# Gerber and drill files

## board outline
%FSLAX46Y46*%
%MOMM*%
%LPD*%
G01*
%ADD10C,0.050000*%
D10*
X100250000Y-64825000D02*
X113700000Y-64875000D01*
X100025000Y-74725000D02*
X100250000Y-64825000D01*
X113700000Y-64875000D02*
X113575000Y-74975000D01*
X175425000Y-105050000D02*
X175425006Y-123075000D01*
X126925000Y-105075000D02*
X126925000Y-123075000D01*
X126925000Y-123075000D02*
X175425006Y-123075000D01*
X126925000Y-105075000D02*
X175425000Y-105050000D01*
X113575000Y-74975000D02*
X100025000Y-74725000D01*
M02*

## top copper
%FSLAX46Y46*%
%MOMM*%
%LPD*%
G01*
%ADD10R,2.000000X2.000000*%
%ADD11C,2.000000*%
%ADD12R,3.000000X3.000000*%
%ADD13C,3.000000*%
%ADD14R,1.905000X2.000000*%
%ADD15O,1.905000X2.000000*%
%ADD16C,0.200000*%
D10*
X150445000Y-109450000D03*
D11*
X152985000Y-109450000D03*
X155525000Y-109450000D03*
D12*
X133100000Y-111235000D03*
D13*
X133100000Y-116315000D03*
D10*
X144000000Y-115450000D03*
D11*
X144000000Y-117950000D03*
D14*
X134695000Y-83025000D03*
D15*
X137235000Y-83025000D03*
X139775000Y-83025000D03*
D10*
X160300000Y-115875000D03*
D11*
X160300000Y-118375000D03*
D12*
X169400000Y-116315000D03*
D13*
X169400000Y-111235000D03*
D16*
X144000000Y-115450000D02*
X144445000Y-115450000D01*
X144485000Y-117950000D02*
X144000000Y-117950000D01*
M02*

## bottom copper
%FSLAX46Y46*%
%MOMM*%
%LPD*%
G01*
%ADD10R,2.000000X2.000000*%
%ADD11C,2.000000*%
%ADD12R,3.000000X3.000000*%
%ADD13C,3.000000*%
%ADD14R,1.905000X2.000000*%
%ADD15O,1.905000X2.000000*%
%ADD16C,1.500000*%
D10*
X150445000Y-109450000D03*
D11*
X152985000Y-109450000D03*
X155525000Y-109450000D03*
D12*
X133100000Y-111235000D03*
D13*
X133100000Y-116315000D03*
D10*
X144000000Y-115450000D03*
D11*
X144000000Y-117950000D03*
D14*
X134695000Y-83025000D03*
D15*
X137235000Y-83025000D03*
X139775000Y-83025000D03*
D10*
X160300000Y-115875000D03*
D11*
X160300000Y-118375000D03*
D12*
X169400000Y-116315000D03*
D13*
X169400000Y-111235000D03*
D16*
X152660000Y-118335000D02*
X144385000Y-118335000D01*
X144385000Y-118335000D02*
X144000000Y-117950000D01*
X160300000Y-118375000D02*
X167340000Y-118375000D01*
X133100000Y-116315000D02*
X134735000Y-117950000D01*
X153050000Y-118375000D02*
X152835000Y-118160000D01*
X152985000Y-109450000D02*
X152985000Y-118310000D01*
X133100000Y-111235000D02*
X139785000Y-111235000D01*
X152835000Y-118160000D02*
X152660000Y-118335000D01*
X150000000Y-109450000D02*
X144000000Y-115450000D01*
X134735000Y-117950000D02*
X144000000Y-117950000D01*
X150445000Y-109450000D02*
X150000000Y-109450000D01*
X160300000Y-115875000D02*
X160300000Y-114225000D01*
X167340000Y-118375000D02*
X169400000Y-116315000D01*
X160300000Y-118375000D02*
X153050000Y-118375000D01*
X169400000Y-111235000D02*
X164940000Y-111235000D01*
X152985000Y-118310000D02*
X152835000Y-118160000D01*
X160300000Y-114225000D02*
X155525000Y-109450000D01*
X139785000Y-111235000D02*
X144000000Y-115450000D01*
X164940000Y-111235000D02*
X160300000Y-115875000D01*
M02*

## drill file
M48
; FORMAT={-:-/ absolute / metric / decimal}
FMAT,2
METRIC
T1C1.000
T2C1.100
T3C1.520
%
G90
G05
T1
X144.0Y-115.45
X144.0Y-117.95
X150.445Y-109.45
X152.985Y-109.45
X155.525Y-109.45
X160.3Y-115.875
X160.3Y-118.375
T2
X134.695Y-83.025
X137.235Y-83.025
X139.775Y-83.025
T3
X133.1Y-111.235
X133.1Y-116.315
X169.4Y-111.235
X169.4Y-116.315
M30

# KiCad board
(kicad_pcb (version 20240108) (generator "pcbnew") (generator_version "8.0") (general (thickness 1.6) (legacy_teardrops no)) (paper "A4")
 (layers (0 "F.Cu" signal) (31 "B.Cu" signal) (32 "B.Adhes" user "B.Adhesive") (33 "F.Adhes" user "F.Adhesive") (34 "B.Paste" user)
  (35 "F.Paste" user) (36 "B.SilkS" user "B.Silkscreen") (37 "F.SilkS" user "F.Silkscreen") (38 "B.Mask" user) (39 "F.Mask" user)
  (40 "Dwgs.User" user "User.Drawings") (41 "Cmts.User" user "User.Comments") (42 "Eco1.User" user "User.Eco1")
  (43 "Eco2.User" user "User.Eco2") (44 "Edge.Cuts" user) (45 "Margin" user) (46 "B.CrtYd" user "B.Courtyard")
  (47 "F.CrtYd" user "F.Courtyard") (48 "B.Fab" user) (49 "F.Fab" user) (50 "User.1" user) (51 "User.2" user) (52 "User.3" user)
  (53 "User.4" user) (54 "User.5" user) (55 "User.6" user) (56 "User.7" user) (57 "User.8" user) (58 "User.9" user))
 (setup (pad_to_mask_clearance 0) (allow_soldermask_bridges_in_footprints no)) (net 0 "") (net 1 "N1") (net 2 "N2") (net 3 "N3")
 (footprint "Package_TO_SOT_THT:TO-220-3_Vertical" (layer "F.Cu") (at 150.445 109.45)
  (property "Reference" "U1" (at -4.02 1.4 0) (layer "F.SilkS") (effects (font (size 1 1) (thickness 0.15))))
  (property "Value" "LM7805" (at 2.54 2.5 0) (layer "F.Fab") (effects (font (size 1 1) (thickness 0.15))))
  (pad "1" thru_hole rect (at 0 0) (size 2 2) (drill 1) (layers "*.Cu" "*.Mask") (remove_unused_layers no))
  (pad "2" thru_hole circle (at 2.54 0) (size 2 2) (drill 1) (layers "*.Cu" "*.Mask") (remove_unused_layers no))
  (pad "3" thru_hole circle (at 5.08 0) (size 2 2) (drill 1) (layers "*.Cu" "*.Mask") (remove_unused_layers no)))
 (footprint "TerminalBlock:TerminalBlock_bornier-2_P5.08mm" (layer "F.Cu") (at 133.1 111.235 -90)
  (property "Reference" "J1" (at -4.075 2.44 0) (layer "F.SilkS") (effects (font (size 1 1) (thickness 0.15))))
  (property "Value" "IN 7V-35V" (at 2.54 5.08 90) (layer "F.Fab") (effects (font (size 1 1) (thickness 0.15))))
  (pad "1" thru_hole rect (at 0 0 270) (size 3 3) (drill 1.52) (layers "*.Cu" "*.Mask") (remove_unused_layers no))
  (pad "2" thru_hole circle (at 5.08 0 270) (size 3 3) (drill 1.52) (layers "*.Cu" "*.Mask") (remove_unused_layers no)))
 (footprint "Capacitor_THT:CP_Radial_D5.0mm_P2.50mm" (layer "F.Cu") (at 144 115.45 -90)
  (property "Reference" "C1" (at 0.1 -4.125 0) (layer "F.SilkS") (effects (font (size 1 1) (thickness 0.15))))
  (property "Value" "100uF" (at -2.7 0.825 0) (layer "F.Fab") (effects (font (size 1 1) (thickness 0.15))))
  (pad "1" thru_hole rect (at 0 0 270) (size 2 2) (drill 1) (layers "*.Cu" "*.Mask") (remove_unused_layers no))
  (pad "2" thru_hole circle (at 2.5 0 270) (size 2 2) (drill 1) (layers "*.Cu" "*.Mask") (remove_unused_layers no)))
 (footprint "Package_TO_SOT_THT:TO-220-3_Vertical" (layer "F.Cu") (at 134.695 83.025)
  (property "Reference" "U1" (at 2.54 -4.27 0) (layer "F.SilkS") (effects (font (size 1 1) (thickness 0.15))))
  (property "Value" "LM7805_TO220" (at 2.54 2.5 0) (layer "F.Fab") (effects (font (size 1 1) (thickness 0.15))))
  (pad "1" thru_hole rect (at 0 0) (size 1.905 2) (drill 1.1) (layers "*.Cu" "*.Mask") (remove_unused_layers no) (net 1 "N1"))
  (pad "2" thru_hole oval (at 2.54 0) (size 1.905 2) (drill 1.1) (layers "*.Cu" "*.Mask") (remove_unused_layers no) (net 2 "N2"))
  (pad "3" thru_hole oval (at 5.08 0) (size 1.905 2) (drill 1.1) (layers "*.Cu" "*.Mask") (remove_unused_layers no) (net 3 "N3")))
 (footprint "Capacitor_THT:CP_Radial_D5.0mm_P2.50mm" (layer "F.Cu") (at 160.3 115.875 -90)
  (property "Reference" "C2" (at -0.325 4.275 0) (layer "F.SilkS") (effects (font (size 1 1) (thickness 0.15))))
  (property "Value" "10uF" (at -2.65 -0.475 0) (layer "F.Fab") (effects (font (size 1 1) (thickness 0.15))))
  (pad "1" thru_hole rect (at 0 0 270) (size 2 2) (drill 1) (layers "*.Cu" "*.Mask") (remove_unused_layers no))
  (pad "2" thru_hole circle (at 2.5 0 270) (size 2 2) (drill 1) (layers "*.Cu" "*.Mask") (remove_unused_layers no)))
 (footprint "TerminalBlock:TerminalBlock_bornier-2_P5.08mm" (layer "F.Cu") (at 169.4 116.315 90)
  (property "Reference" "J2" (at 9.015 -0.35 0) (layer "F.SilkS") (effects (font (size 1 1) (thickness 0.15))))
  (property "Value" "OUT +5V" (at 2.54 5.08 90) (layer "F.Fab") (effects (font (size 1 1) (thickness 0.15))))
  (pad "1" thru_hole rect (at 0 0 90) (size 3 3) (drill 1.52) (layers "*.Cu" "*.Mask") (remove_unused_layers no))
  (pad "2" thru_hole circle (at 5.08 0 90) (size 3 3) (drill 1.52) (layers "*.Cu" "*.Mask") (remove_unused_layers no)))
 (gr_line (start 100.25 64.825) (end 113.7 64.875) (stroke (width 0.05) (type default)) (layer "Edge.Cuts"))
 (gr_line (start 100.025 74.725) (end 100.25 64.825) (stroke (width 0.05) (type default)) (layer "Edge.Cuts"))
 (gr_line (start 113.7 64.875) (end 113.575 74.975) (stroke (width 0.05) (type default)) (layer "Edge.Cuts"))
 (gr_line (start 175.425 105.05) (end 175.425006 123.075) (stroke (width 0.05) (type default)) (layer "Edge.Cuts"))
 (gr_line (start 126.925 105.075) (end 126.925 123.075) (stroke (width 0.05) (type default)) (layer "Edge.Cuts"))
 (gr_line (start 126.925 123.075) (end 175.425006 123.075) (stroke (width 0.05) (type default)) (layer "Edge.Cuts"))
 (gr_line (start 126.925 105.075) (end 175.425 105.05) (stroke (width 0.05) (type default)) (layer "Edge.Cuts"))
 (gr_line (start 113.575 74.975) (end 100.025 74.725) (stroke (width 0.05) (type default)) (layer "Edge.Cuts"))
 (segment (start 144 115.45) (end 144.445 115.45) (width 0.2) (layer "F.Cu") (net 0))
 (segment (start 144.485 117.95) (end 144 117.95) (width 0.2) (layer "F.Cu") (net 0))
 (segment (start 152.66 118.335) (end 144.385 118.335) (width 1.5) (layer "B.Cu") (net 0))
 (segment (start 144.385 118.335) (end 144 117.95) (width 1.5) (layer "B.Cu") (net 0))
 (segment (start 160.3 118.375) (end 167.34 118.375) (width 1.5) (layer "B.Cu") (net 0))
 (segment (start 133.1 116.315) (end 134.735 117.95) (width 1.5) (layer "B.Cu") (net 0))
 (segment (start 153.05 118.375) (end 152.835 118.16) (width 1.5) (layer "B.Cu") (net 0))
 (segment (start 152.985 109.45) (end 152.985 118.31) (width 1.5) (layer "B.Cu") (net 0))
 (segment (start 133.1 111.235) (end 139.785 111.235) (width 1.5) (layer "B.Cu") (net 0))
 (segment (start 152.835 118.16) (end 152.66 118.335) (width 1.5) (layer "B.Cu") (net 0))
 (segment (start 150 109.45) (end 144 115.45) (width 1.5) (layer "B.Cu") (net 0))
 (segment (start 134.735 117.95) (end 144 117.95) (width 1.5) (layer "B.Cu") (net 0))
 (segment (start 150.445 109.45) (end 150 109.45) (width 1.5) (layer "B.Cu") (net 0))
 (segment (start 160.3 115.875) (end 160.3 114.225) (width 1.5) (layer "B.Cu") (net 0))
 (segment (start 167.34 118.375) (end 169.4 116.315) (width 1.5) (layer "B.Cu") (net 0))
 (segment (start 160.3 118.375) (end 153.05 118.375) (width 1.5) (layer "B.Cu") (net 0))
 (segment (start 169.4 111.235) (end 164.94 111.235) (width 1.5) (layer "B.Cu") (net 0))
 (segment (start 152.985 118.31) (end 152.835 118.16) (width 1.5) (layer "B.Cu") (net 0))
 (segment (start 160.3 114.225) (end 155.525 109.45) (width 1.5) (layer "B.Cu") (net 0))
 (segment (start 139.785 111.235) (end 144 115.45) (width 1.5) (layer "B.Cu") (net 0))
 (segment (start 164.94 111.235) (end 160.3 115.875) (width 1.5) (layer "B.Cu") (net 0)))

